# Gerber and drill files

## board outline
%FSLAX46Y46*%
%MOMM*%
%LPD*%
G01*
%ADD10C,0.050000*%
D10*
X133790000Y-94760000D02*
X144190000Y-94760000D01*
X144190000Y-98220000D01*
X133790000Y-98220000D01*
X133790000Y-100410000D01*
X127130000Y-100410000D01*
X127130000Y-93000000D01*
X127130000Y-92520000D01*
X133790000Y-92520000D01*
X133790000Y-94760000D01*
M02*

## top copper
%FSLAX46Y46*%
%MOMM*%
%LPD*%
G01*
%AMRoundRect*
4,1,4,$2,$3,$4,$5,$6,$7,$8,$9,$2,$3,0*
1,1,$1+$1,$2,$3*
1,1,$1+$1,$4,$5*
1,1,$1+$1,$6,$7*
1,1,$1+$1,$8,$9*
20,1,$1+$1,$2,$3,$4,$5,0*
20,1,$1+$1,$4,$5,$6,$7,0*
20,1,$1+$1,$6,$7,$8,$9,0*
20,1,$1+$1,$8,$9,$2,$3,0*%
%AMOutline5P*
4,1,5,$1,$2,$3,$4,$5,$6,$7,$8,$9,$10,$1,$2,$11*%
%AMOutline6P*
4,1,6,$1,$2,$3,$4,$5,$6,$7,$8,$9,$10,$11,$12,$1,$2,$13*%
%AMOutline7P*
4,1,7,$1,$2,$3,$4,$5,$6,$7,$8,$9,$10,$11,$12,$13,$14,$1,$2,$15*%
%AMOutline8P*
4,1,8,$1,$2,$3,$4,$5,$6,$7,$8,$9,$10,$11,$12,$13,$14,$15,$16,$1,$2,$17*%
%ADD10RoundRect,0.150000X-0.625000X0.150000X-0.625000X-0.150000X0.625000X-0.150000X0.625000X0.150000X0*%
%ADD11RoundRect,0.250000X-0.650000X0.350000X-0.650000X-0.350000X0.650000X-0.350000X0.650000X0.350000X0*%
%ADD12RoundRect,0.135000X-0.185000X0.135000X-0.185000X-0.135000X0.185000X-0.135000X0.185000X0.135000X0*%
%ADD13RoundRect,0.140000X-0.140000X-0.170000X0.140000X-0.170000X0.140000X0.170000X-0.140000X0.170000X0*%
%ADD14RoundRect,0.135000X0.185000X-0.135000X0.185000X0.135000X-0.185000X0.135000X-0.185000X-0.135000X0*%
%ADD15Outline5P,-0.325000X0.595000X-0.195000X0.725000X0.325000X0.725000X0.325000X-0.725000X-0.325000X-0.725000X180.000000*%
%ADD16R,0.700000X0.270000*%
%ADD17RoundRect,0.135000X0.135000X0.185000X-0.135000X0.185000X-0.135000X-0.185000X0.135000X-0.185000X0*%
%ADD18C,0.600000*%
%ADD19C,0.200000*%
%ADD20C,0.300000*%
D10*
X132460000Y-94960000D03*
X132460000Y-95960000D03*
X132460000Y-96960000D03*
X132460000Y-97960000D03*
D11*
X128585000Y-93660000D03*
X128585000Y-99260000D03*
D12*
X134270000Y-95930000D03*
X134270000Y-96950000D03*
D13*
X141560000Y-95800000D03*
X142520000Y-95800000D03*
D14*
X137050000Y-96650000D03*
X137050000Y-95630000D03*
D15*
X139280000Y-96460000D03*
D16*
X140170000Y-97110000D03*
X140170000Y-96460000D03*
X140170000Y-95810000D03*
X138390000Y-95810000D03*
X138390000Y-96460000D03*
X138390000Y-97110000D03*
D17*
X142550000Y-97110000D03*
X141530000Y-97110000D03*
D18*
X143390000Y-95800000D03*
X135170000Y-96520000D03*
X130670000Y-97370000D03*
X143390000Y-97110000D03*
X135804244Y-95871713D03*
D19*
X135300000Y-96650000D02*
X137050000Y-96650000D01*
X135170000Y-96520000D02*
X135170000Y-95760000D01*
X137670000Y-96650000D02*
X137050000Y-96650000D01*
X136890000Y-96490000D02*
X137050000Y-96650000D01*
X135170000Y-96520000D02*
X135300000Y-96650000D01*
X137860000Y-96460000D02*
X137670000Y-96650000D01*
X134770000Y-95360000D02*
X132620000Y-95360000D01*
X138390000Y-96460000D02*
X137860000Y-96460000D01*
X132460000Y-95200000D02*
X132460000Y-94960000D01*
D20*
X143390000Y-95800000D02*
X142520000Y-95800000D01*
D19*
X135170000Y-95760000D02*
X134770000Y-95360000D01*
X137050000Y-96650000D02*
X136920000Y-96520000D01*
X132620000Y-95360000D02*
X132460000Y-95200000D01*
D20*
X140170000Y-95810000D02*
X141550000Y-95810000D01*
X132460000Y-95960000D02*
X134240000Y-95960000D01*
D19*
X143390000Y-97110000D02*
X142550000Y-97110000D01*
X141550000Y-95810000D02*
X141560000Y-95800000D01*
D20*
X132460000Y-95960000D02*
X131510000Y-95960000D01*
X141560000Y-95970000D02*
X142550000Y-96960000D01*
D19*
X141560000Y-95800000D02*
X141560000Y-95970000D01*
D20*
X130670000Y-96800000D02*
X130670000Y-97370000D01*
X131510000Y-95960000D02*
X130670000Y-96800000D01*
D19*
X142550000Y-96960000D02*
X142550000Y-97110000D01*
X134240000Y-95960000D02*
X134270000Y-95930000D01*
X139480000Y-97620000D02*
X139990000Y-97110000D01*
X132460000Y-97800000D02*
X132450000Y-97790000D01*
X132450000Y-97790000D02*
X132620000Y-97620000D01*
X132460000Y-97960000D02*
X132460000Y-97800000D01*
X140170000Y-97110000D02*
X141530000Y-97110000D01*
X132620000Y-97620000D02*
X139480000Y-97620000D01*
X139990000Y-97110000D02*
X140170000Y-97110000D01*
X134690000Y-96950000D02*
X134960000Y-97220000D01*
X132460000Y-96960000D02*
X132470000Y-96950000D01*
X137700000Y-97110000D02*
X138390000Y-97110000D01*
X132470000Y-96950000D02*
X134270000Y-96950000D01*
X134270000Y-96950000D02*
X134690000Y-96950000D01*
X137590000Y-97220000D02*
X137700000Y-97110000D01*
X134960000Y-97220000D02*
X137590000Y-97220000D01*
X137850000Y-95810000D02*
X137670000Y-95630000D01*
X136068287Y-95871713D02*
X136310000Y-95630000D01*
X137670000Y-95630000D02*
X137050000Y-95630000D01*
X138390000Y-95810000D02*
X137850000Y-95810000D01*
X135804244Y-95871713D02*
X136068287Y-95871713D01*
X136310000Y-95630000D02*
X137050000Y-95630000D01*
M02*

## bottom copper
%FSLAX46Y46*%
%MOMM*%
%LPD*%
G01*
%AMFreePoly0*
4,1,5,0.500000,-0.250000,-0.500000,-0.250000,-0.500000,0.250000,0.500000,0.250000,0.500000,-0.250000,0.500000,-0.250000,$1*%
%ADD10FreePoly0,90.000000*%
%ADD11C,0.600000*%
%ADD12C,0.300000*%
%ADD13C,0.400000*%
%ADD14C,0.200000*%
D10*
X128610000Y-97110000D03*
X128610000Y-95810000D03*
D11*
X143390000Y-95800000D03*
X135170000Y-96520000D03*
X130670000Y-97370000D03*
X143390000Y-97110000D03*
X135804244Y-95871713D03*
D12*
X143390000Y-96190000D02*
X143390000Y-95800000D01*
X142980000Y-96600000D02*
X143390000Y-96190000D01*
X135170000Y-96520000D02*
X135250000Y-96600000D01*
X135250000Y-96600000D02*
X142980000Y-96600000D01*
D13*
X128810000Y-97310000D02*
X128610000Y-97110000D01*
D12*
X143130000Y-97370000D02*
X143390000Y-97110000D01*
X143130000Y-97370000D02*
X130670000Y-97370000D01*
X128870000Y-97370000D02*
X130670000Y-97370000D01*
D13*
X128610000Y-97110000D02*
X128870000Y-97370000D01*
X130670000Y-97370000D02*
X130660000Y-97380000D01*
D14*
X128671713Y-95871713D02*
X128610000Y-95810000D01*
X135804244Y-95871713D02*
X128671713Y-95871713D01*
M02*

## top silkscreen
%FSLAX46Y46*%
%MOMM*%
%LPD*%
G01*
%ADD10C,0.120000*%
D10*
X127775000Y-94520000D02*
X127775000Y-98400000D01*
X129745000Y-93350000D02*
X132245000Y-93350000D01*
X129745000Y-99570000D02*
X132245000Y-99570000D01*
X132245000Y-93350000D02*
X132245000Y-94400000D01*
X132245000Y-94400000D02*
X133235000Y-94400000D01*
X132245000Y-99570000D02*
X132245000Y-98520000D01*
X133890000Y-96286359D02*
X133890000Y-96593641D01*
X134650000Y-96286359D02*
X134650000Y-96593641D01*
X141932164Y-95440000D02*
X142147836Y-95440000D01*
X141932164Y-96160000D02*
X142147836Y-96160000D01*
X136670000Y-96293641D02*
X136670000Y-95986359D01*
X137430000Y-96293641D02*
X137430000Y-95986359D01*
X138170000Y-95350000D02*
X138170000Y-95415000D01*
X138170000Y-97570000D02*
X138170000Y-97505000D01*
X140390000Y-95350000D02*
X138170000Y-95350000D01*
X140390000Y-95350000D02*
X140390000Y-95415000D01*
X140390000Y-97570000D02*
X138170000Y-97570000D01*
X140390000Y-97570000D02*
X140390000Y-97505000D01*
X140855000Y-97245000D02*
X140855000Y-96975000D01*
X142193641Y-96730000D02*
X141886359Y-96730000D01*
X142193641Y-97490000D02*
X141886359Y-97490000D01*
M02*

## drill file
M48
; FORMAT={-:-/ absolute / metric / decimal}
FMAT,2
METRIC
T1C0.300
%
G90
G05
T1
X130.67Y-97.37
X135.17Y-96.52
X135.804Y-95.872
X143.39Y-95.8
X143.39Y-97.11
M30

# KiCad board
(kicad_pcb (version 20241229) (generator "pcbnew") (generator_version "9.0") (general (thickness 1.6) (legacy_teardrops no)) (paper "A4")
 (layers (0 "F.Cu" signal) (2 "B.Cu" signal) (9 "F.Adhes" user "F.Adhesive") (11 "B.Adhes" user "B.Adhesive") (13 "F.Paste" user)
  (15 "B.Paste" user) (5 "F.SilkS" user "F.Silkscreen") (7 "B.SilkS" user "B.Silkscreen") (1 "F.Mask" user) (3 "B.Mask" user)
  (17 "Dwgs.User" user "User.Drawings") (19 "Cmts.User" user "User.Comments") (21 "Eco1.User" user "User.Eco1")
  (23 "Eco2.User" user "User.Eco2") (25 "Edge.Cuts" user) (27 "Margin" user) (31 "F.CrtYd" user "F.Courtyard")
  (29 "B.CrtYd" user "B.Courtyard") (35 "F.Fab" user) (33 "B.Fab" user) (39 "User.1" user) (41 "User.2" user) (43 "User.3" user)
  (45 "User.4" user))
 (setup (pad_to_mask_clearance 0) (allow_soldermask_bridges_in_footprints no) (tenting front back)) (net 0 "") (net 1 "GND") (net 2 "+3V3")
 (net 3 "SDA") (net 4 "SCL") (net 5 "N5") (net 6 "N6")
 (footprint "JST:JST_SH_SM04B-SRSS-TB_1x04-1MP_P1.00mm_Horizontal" (layer "F.Cu") (at 130.46 96.46 -90)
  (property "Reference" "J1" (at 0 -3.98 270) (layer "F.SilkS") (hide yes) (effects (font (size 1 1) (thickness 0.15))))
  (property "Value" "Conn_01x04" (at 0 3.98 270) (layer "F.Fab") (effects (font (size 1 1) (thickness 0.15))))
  (fp_line (start -1.94 2.685) (end 1.94 2.685) (stroke (width 0.12) (type solid)) (layer "F.SilkS"))
  (fp_line (start -3.11 0.715) (end -3.11 -1.785) (stroke (width 0.12) (type solid)) (layer "F.SilkS"))
  (fp_line (start 3.11 0.715) (end 3.11 -1.785) (stroke (width 0.12) (type solid)) (layer "F.SilkS"))
  (fp_line (start -3.11 -1.785) (end -2.06 -1.785) (stroke (width 0.12) (type solid)) (layer "F.SilkS"))
  (fp_line (start -2.06 -1.785) (end -2.06 -2.775) (stroke (width 0.12) (type solid)) (layer "F.SilkS"))
  (fp_line (start 3.11 -1.785) (end 2.06 -1.785) (stroke (width 0.12) (type solid)) (layer "F.SilkS"))
  (pad "1" smd roundrect (at -1.5 -2 270) (size 0.6 1.55) (layers "F.Cu" "F.Mask" "F.Paste") (roundrect_rratio 0.25) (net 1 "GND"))
  (pad "2" smd roundrect (at -0.5 -2 270) (size 0.6 1.55) (layers "F.Cu" "F.Mask" "F.Paste") (roundrect_rratio 0.25) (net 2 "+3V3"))
  (pad "3" smd roundrect (at 0.5 -2 270) (size 0.6 1.55) (layers "F.Cu" "F.Mask" "F.Paste") (roundrect_rratio 0.25) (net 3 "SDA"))
  (pad "4" smd roundrect (at 1.5 -2 270) (size 0.6 1.55) (layers "F.Cu" "F.Mask" "F.Paste") (roundrect_rratio 0.25) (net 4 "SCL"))
  (pad "MP" smd roundrect (at -2.8 1.875 270) (size 1.2 1.8) (layers "F.Cu" "F.Mask" "F.Paste") (roundrect_rratio 0.208333))
  (pad "MP" smd roundrect (at 2.8 1.875 270) (size 1.2 1.8) (layers "F.Cu" "F.Mask" "F.Paste") (roundrect_rratio 0.208333)))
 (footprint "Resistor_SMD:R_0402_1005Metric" (layer "F.Cu") (at 134.27 96.44 -90)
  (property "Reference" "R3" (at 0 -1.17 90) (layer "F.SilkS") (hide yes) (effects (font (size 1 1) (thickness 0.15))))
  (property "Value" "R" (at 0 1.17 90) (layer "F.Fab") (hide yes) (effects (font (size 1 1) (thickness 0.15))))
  (fp_line (start -0.153641 0.38) (end 0.153641 0.38) (stroke (width 0.12) (type solid)) (layer "F.SilkS"))
  (fp_line (start -0.153641 -0.38) (end 0.153641 -0.38) (stroke (width 0.12) (type solid)) (layer "F.SilkS"))
  (pad "1" smd roundrect (at -0.51 0 270) (size 0.54 0.64) (layers "F.Cu" "F.Mask" "F.Paste") (roundrect_rratio 0.25) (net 2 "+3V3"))
  (pad "2" smd roundrect (at 0.51 0 270) (size 0.54 0.64) (layers "F.Cu" "F.Mask" "F.Paste") (roundrect_rratio 0.25) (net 3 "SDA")))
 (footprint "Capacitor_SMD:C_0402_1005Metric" (layer "F.Cu") (at 142.04 95.8)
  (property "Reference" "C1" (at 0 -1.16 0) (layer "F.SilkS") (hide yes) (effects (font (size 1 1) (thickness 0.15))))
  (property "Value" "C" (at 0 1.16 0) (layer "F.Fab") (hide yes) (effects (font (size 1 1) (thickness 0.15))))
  (fp_line (start -0.107836 -0.36) (end 0.107836 -0.36) (stroke (width 0.12) (type solid)) (layer "F.SilkS"))
  (fp_line (start -0.107836 0.36) (end 0.107836 0.36) (stroke (width 0.12) (type solid)) (layer "F.SilkS"))
  (pad "1" smd roundrect (at -0.48 0) (size 0.56 0.62) (layers "F.Cu" "F.Mask" "F.Paste") (roundrect_rratio 0.25) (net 2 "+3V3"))
  (pad "2" smd roundrect (at 0.48 0) (size 0.56 0.62) (layers "F.Cu" "F.Mask" "F.Paste") (roundrect_rratio 0.25) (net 1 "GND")))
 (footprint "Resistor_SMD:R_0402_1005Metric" (layer "F.Cu") (at 137.05 96.14 90)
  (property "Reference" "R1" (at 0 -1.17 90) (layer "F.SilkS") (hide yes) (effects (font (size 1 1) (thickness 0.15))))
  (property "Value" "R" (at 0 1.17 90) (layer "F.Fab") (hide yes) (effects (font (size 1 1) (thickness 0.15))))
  (fp_line (start -0.153641 -0.38) (end 0.153641 -0.38) (stroke (width 0.12) (type solid)) (layer "F.SilkS"))
  (fp_line (start -0.153641 0.38) (end 0.153641 0.38) (stroke (width 0.12) (type solid)) (layer "F.SilkS"))
  (pad "1" smd roundrect (at -0.51 0 90) (size 0.54 0.64) (layers "F.Cu" "F.Mask" "F.Paste") (roundrect_rratio 0.25) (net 1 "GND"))
  (pad "2" smd roundrect (at 0.51 0 90) (size 0.54 0.64) (layers "F.Cu" "F.Mask" "F.Paste") (roundrect_rratio 0.25) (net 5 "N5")))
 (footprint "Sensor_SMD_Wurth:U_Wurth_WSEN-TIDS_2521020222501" (layer "F.Cu") (at 139.28 96.46 180)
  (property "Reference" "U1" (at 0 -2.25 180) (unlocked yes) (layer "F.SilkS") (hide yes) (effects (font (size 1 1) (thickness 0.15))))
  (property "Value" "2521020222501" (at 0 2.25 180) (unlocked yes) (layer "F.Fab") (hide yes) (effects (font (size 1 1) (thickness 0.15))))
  (fp_line (start 1.11 1.11) (end 1.11 1.045) (stroke (width 0.12) (type solid)) (layer "F.SilkS"))
  (fp_line (start 1.11 -1.11) (end 1.11 -1.045) (stroke (width 0.12) (type solid)) (layer "F.SilkS"))
  (fp_line (start -1.11 1.11) (end 1.11 1.11) (stroke (width 0.12) (type solid)) (layer "F.SilkS"))
  (fp_line (start -1.11 1.11) (end -1.11 1.045) (stroke (width 0.12) (type solid)) (layer "F.SilkS"))
  (fp_line (start -1.11 -1.11) (end 1.11 -1.11) (stroke (width 0.12) (type solid)) (layer "F.SilkS"))
  (fp_line (start -1.11 -1.11) (end -1.11 -1.045) (stroke (width 0.12) (type solid)) (layer "F.SilkS"))
  (fp_line (start -1.575 -0.785) (end -1.575 -0.515) (stroke (width 0.12) (type solid)) (layer "F.SilkS"))
  (pad "" smd roundrect (at 0 0 180) (size 0.65 1.45) (layers "F.Cu" "F.Mask" "F.Paste") (roundrect_rratio 0) (chamfer_ratio 0.2)
   (chamfer top_left))
  (pad "1" smd rect (at -0.89 -0.65 180) (size 0.7 0.27) (layers "F.Cu" "F.Mask" "F.Paste") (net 4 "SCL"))
  (pad "2" smd rect (at -0.89 0 180) (size 0.7 0.27) (layers "F.Cu" "F.Mask" "F.Paste") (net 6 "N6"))
  (pad "3" smd rect (at -0.89 0.65 180) (size 0.7 0.27) (layers "F.Cu" "F.Mask" "F.Paste") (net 2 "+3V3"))
  (pad "4" smd rect (at 0.89 0.65 180) (size 0.7 0.27) (layers "F.Cu" "F.Mask" "F.Paste") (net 5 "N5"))
  (pad "5" smd rect (at 0.89 0 180) (size 0.7 0.27) (layers "F.Cu" "F.Mask" "F.Paste") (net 1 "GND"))
  (pad "6" smd rect (at 0.89 -0.65 180) (size 0.7 0.27) (layers "F.Cu" "F.Mask" "F.Paste") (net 3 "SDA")))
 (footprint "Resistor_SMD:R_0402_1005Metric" (layer "F.Cu") (at 142.04 97.11 180)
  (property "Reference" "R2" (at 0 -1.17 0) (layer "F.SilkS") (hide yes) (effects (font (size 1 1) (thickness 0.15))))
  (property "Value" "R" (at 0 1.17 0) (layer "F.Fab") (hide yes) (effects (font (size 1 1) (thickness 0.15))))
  (fp_line (start -0.153641 0.38) (end 0.153641 0.38) (stroke (width 0.12) (type solid)) (layer "F.SilkS"))
  (fp_line (start -0.153641 -0.38) (end 0.153641 -0.38) (stroke (width 0.12) (type solid)) (layer "F.SilkS"))
  (pad "1" smd roundrect (at -0.51 0 180) (size 0.54 0.64) (layers "F.Cu" "F.Mask" "F.Paste") (roundrect_rratio 0.25) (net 2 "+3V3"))
  (pad "2" smd roundrect (at 0.51 0 180) (size 0.54 0.64) (layers "F.Cu" "F.Mask" "F.Paste") (roundrect_rratio 0.25) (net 4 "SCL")))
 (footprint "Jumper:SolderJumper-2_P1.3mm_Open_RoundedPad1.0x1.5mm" (layer "B.Cu") (at 128.61 96.46 90)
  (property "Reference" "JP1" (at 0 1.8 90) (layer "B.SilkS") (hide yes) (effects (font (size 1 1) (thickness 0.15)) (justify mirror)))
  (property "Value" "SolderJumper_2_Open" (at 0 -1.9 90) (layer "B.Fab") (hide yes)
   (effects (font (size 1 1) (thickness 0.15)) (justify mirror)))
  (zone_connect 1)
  (pad "1" smd custom (at -0.65 0 90) (size 1 0.5) (layers "B.Cu" "B.Mask") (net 2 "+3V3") (zone_connect 2) (thermal_bridge_angle 45)
   (options (clearance outline) (anchor rect)) (primitives))
  (pad "2" smd custom (at 0.65 0 90) (size 1 0.5) (layers "B.Cu" "B.Mask") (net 5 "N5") (zone_connect 2) (thermal_bridge_angle 45)
   (options (clearance outline) (anchor rect)) (primitives)))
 (gr_poly
  (pts (xy 133.79 94.76) (xy 144.19 94.76) (xy 144.19 98.22) (xy 133.79 98.22) (xy 133.79 100.41) (xy 127.13 100.41) (xy 127.13 93)
   (xy 127.13 92.52) (xy 133.79 92.52))
  (stroke (width 0.05) (type solid)) (fill no) (layer "Edge.Cuts"))
 (segment (start 135.3 96.65) (end 137.05 96.65) (width 0.2) (layer "F.Cu") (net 1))
 (segment (start 135.17 96.52) (end 135.17 95.76) (width 0.2) (layer "F.Cu") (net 1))
 (segment (start 137.67 96.65) (end 137.05 96.65) (width 0.2) (layer "F.Cu") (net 1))
 (segment (start 136.89 96.49) (end 137.05 96.65) (width 0.2) (layer "F.Cu") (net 1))
 (segment (start 135.17 96.52) (end 135.3 96.65) (width 0.2) (layer "F.Cu") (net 1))
 (segment (start 137.86 96.46) (end 137.67 96.65) (width 0.2) (layer "F.Cu") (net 1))
 (segment (start 134.77 95.36) (end 132.62 95.36) (width 0.2) (layer "F.Cu") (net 1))
 (segment (start 138.39 96.46) (end 137.86 96.46) (width 0.2) (layer "F.Cu") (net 1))
 (segment (start 132.46 95.2) (end 132.46 94.96) (width 0.2) (layer "F.Cu") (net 1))
 (segment (start 143.39 95.8) (end 142.52 95.8) (width 0.3) (layer "F.Cu") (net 1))
 (segment (start 135.17 95.76) (end 134.77 95.36) (width 0.2) (layer "F.Cu") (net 1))
 (segment (start 137.05 96.65) (end 136.92 96.52) (width 0.2) (layer "F.Cu") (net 1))
 (segment (start 132.62 95.36) (end 132.46 95.2) (width 0.2) (layer "F.Cu") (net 1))
 (via (at 143.39 95.8) (size 0.6) (drill 0.3) (layers "F.Cu" "B.Cu") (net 1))
 (via (at 135.17 96.52) (size 0.6) (drill 0.3) (layers "F.Cu" "B.Cu") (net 1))
 (segment (start 143.39 96.19) (end 143.39 95.8) (width 0.3) (layer "B.Cu") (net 1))
 (segment (start 142.98 96.6) (end 143.39 96.19) (width 0.3) (layer "B.Cu") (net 1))
 (segment (start 135.17 96.52) (end 135.25 96.6) (width 0.3) (layer "B.Cu") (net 1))
 (segment (start 135.25 96.6) (end 142.98 96.6) (width 0.3) (layer "B.Cu") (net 1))
 (segment (start 140.17 95.81) (end 141.55 95.81) (width 0.3) (layer "F.Cu") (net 2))
 (segment (start 132.46 95.96) (end 134.24 95.96) (width 0.3) (layer "F.Cu") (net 2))
 (segment (start 143.39 97.11) (end 142.55 97.11) (width 0.2) (layer "F.Cu") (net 2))
 (segment (start 141.55 95.81) (end 141.56 95.8) (width 0.2) (layer "F.Cu") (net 2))
 (segment (start 132.46 95.96) (end 131.51 95.96) (width 0.3) (layer "F.Cu") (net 2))
 (segment (start 141.56 95.97) (end 142.55 96.96) (width 0.3) (layer "F.Cu") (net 2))
 (segment (start 141.56 95.8) (end 141.56 95.97) (width 0.2) (layer "F.Cu") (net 2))
 (segment (start 130.67 96.8) (end 130.67 97.37) (width 0.3) (layer "F.Cu") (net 2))
 (segment (start 131.51 95.96) (end 130.67 96.8) (width 0.3) (layer "F.Cu") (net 2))
 (segment (start 142.55 96.96) (end 142.55 97.11) (width 0.2) (layer "F.Cu") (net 2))
 (segment (start 134.24 95.96) (end 134.27 95.93) (width 0.2) (layer "F.Cu") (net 2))
 (via (at 130.67 97.37) (size 0.6) (drill 0.3) (layers "F.Cu" "B.Cu") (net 2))
 (via (at 143.39 97.11) (size 0.6) (drill 0.3) (layers "F.Cu" "B.Cu") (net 2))
 (segment (start 128.81 97.31) (end 128.61 97.11) (width 0.4) (layer "B.Cu") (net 2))
 (segment (start 143.13 97.37) (end 143.39 97.11) (width 0.3) (layer "B.Cu") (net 2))
 (segment (start 143.13 97.37) (end 130.67 97.37) (width 0.3) (layer "B.Cu") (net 2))
 (segment (start 128.87 97.37) (end 130.67 97.37) (width 0.3) (layer "B.Cu") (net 2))
 (segment (start 128.61 97.11) (end 128.87 97.37) (width 0.4) (layer "B.Cu") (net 2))
 (segment (start 130.67 97.37) (end 130.66 97.38) (width 0.4) (layer "B.Cu") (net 2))
 (segment (start 139.48 97.62) (end 139.99 97.11) (width 0.2) (layer "F.Cu") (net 4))
 (segment (start 132.46 97.8) (end 132.45 97.79) (width 0.2) (layer "F.Cu") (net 4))
 (segment (start 132.45 97.79) (end 132.62 97.62) (width 0.2) (layer "F.Cu") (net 4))
 (segment (start 132.46 97.96) (end 132.46 97.8) (width 0.2) (layer "F.Cu") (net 4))
 (segment (start 140.17 97.11) (end 141.53 97.11) (width 0.2) (layer "F.Cu") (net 4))
 (segment (start 132.62 97.62) (end 139.48 97.62) (width 0.2) (layer "F.Cu") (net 4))
 (segment (start 139.99 97.11) (end 140.17 97.11) (width 0.2) (layer "F.Cu") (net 4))
 (segment (start 134.69 96.95) (end 134.96 97.22) (width 0.2) (layer "F.Cu") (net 3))
 (segment (start 132.46 96.96) (end 132.47 96.95) (width 0.2) (layer "F.Cu") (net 3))
 (segment (start 137.7 97.11) (end 138.39 97.11) (width 0.2) (layer "F.Cu") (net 3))
 (segment (start 132.47 96.95) (end 134.27 96.95) (width 0.2) (layer "F.Cu") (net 3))
 (segment (start 134.27 96.95) (end 134.69 96.95) (width 0.2) (layer "F.Cu") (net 3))
 (segment (start 137.59 97.22) (end 137.7 97.11) (width 0.2) (layer "F.Cu") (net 3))
 (segment (start 134.96 97.22) (end 137.59 97.22) (width 0.2) (layer "F.Cu") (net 3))
 (segment (start 137.85 95.81) (end 137.67 95.63) (width 0.2) (layer "F.Cu") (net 5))
 (segment (start 136.068287 95.871713) (end 136.31 95.63) (width 0.2) (layer "F.Cu") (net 5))
 (segment (start 137.67 95.63) (end 137.05 95.63) (width 0.2) (layer "F.Cu") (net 5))
 (segment (start 138.39 95.81) (end 137.85 95.81) (width 0.2) (layer "F.Cu") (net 5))
 (segment (start 135.804244 95.871713) (end 136.068287 95.871713) (width 0.2) (layer "F.Cu") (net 5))
 (segment (start 136.31 95.63) (end 137.05 95.63) (width 0.2) (layer "F.Cu") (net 5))
 (via (at 135.804244 95.871713) (size 0.6) (drill 0.3) (layers "F.Cu" "B.Cu") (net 5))
 (segment (start 128.671713 95.871713) (end 128.61 95.81) (width 0.2) (layer "B.Cu") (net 5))
 (segment (start 135.804244 95.871713) (end 128.671713 95.871713) (width 0.2) (layer "B.Cu") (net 5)))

